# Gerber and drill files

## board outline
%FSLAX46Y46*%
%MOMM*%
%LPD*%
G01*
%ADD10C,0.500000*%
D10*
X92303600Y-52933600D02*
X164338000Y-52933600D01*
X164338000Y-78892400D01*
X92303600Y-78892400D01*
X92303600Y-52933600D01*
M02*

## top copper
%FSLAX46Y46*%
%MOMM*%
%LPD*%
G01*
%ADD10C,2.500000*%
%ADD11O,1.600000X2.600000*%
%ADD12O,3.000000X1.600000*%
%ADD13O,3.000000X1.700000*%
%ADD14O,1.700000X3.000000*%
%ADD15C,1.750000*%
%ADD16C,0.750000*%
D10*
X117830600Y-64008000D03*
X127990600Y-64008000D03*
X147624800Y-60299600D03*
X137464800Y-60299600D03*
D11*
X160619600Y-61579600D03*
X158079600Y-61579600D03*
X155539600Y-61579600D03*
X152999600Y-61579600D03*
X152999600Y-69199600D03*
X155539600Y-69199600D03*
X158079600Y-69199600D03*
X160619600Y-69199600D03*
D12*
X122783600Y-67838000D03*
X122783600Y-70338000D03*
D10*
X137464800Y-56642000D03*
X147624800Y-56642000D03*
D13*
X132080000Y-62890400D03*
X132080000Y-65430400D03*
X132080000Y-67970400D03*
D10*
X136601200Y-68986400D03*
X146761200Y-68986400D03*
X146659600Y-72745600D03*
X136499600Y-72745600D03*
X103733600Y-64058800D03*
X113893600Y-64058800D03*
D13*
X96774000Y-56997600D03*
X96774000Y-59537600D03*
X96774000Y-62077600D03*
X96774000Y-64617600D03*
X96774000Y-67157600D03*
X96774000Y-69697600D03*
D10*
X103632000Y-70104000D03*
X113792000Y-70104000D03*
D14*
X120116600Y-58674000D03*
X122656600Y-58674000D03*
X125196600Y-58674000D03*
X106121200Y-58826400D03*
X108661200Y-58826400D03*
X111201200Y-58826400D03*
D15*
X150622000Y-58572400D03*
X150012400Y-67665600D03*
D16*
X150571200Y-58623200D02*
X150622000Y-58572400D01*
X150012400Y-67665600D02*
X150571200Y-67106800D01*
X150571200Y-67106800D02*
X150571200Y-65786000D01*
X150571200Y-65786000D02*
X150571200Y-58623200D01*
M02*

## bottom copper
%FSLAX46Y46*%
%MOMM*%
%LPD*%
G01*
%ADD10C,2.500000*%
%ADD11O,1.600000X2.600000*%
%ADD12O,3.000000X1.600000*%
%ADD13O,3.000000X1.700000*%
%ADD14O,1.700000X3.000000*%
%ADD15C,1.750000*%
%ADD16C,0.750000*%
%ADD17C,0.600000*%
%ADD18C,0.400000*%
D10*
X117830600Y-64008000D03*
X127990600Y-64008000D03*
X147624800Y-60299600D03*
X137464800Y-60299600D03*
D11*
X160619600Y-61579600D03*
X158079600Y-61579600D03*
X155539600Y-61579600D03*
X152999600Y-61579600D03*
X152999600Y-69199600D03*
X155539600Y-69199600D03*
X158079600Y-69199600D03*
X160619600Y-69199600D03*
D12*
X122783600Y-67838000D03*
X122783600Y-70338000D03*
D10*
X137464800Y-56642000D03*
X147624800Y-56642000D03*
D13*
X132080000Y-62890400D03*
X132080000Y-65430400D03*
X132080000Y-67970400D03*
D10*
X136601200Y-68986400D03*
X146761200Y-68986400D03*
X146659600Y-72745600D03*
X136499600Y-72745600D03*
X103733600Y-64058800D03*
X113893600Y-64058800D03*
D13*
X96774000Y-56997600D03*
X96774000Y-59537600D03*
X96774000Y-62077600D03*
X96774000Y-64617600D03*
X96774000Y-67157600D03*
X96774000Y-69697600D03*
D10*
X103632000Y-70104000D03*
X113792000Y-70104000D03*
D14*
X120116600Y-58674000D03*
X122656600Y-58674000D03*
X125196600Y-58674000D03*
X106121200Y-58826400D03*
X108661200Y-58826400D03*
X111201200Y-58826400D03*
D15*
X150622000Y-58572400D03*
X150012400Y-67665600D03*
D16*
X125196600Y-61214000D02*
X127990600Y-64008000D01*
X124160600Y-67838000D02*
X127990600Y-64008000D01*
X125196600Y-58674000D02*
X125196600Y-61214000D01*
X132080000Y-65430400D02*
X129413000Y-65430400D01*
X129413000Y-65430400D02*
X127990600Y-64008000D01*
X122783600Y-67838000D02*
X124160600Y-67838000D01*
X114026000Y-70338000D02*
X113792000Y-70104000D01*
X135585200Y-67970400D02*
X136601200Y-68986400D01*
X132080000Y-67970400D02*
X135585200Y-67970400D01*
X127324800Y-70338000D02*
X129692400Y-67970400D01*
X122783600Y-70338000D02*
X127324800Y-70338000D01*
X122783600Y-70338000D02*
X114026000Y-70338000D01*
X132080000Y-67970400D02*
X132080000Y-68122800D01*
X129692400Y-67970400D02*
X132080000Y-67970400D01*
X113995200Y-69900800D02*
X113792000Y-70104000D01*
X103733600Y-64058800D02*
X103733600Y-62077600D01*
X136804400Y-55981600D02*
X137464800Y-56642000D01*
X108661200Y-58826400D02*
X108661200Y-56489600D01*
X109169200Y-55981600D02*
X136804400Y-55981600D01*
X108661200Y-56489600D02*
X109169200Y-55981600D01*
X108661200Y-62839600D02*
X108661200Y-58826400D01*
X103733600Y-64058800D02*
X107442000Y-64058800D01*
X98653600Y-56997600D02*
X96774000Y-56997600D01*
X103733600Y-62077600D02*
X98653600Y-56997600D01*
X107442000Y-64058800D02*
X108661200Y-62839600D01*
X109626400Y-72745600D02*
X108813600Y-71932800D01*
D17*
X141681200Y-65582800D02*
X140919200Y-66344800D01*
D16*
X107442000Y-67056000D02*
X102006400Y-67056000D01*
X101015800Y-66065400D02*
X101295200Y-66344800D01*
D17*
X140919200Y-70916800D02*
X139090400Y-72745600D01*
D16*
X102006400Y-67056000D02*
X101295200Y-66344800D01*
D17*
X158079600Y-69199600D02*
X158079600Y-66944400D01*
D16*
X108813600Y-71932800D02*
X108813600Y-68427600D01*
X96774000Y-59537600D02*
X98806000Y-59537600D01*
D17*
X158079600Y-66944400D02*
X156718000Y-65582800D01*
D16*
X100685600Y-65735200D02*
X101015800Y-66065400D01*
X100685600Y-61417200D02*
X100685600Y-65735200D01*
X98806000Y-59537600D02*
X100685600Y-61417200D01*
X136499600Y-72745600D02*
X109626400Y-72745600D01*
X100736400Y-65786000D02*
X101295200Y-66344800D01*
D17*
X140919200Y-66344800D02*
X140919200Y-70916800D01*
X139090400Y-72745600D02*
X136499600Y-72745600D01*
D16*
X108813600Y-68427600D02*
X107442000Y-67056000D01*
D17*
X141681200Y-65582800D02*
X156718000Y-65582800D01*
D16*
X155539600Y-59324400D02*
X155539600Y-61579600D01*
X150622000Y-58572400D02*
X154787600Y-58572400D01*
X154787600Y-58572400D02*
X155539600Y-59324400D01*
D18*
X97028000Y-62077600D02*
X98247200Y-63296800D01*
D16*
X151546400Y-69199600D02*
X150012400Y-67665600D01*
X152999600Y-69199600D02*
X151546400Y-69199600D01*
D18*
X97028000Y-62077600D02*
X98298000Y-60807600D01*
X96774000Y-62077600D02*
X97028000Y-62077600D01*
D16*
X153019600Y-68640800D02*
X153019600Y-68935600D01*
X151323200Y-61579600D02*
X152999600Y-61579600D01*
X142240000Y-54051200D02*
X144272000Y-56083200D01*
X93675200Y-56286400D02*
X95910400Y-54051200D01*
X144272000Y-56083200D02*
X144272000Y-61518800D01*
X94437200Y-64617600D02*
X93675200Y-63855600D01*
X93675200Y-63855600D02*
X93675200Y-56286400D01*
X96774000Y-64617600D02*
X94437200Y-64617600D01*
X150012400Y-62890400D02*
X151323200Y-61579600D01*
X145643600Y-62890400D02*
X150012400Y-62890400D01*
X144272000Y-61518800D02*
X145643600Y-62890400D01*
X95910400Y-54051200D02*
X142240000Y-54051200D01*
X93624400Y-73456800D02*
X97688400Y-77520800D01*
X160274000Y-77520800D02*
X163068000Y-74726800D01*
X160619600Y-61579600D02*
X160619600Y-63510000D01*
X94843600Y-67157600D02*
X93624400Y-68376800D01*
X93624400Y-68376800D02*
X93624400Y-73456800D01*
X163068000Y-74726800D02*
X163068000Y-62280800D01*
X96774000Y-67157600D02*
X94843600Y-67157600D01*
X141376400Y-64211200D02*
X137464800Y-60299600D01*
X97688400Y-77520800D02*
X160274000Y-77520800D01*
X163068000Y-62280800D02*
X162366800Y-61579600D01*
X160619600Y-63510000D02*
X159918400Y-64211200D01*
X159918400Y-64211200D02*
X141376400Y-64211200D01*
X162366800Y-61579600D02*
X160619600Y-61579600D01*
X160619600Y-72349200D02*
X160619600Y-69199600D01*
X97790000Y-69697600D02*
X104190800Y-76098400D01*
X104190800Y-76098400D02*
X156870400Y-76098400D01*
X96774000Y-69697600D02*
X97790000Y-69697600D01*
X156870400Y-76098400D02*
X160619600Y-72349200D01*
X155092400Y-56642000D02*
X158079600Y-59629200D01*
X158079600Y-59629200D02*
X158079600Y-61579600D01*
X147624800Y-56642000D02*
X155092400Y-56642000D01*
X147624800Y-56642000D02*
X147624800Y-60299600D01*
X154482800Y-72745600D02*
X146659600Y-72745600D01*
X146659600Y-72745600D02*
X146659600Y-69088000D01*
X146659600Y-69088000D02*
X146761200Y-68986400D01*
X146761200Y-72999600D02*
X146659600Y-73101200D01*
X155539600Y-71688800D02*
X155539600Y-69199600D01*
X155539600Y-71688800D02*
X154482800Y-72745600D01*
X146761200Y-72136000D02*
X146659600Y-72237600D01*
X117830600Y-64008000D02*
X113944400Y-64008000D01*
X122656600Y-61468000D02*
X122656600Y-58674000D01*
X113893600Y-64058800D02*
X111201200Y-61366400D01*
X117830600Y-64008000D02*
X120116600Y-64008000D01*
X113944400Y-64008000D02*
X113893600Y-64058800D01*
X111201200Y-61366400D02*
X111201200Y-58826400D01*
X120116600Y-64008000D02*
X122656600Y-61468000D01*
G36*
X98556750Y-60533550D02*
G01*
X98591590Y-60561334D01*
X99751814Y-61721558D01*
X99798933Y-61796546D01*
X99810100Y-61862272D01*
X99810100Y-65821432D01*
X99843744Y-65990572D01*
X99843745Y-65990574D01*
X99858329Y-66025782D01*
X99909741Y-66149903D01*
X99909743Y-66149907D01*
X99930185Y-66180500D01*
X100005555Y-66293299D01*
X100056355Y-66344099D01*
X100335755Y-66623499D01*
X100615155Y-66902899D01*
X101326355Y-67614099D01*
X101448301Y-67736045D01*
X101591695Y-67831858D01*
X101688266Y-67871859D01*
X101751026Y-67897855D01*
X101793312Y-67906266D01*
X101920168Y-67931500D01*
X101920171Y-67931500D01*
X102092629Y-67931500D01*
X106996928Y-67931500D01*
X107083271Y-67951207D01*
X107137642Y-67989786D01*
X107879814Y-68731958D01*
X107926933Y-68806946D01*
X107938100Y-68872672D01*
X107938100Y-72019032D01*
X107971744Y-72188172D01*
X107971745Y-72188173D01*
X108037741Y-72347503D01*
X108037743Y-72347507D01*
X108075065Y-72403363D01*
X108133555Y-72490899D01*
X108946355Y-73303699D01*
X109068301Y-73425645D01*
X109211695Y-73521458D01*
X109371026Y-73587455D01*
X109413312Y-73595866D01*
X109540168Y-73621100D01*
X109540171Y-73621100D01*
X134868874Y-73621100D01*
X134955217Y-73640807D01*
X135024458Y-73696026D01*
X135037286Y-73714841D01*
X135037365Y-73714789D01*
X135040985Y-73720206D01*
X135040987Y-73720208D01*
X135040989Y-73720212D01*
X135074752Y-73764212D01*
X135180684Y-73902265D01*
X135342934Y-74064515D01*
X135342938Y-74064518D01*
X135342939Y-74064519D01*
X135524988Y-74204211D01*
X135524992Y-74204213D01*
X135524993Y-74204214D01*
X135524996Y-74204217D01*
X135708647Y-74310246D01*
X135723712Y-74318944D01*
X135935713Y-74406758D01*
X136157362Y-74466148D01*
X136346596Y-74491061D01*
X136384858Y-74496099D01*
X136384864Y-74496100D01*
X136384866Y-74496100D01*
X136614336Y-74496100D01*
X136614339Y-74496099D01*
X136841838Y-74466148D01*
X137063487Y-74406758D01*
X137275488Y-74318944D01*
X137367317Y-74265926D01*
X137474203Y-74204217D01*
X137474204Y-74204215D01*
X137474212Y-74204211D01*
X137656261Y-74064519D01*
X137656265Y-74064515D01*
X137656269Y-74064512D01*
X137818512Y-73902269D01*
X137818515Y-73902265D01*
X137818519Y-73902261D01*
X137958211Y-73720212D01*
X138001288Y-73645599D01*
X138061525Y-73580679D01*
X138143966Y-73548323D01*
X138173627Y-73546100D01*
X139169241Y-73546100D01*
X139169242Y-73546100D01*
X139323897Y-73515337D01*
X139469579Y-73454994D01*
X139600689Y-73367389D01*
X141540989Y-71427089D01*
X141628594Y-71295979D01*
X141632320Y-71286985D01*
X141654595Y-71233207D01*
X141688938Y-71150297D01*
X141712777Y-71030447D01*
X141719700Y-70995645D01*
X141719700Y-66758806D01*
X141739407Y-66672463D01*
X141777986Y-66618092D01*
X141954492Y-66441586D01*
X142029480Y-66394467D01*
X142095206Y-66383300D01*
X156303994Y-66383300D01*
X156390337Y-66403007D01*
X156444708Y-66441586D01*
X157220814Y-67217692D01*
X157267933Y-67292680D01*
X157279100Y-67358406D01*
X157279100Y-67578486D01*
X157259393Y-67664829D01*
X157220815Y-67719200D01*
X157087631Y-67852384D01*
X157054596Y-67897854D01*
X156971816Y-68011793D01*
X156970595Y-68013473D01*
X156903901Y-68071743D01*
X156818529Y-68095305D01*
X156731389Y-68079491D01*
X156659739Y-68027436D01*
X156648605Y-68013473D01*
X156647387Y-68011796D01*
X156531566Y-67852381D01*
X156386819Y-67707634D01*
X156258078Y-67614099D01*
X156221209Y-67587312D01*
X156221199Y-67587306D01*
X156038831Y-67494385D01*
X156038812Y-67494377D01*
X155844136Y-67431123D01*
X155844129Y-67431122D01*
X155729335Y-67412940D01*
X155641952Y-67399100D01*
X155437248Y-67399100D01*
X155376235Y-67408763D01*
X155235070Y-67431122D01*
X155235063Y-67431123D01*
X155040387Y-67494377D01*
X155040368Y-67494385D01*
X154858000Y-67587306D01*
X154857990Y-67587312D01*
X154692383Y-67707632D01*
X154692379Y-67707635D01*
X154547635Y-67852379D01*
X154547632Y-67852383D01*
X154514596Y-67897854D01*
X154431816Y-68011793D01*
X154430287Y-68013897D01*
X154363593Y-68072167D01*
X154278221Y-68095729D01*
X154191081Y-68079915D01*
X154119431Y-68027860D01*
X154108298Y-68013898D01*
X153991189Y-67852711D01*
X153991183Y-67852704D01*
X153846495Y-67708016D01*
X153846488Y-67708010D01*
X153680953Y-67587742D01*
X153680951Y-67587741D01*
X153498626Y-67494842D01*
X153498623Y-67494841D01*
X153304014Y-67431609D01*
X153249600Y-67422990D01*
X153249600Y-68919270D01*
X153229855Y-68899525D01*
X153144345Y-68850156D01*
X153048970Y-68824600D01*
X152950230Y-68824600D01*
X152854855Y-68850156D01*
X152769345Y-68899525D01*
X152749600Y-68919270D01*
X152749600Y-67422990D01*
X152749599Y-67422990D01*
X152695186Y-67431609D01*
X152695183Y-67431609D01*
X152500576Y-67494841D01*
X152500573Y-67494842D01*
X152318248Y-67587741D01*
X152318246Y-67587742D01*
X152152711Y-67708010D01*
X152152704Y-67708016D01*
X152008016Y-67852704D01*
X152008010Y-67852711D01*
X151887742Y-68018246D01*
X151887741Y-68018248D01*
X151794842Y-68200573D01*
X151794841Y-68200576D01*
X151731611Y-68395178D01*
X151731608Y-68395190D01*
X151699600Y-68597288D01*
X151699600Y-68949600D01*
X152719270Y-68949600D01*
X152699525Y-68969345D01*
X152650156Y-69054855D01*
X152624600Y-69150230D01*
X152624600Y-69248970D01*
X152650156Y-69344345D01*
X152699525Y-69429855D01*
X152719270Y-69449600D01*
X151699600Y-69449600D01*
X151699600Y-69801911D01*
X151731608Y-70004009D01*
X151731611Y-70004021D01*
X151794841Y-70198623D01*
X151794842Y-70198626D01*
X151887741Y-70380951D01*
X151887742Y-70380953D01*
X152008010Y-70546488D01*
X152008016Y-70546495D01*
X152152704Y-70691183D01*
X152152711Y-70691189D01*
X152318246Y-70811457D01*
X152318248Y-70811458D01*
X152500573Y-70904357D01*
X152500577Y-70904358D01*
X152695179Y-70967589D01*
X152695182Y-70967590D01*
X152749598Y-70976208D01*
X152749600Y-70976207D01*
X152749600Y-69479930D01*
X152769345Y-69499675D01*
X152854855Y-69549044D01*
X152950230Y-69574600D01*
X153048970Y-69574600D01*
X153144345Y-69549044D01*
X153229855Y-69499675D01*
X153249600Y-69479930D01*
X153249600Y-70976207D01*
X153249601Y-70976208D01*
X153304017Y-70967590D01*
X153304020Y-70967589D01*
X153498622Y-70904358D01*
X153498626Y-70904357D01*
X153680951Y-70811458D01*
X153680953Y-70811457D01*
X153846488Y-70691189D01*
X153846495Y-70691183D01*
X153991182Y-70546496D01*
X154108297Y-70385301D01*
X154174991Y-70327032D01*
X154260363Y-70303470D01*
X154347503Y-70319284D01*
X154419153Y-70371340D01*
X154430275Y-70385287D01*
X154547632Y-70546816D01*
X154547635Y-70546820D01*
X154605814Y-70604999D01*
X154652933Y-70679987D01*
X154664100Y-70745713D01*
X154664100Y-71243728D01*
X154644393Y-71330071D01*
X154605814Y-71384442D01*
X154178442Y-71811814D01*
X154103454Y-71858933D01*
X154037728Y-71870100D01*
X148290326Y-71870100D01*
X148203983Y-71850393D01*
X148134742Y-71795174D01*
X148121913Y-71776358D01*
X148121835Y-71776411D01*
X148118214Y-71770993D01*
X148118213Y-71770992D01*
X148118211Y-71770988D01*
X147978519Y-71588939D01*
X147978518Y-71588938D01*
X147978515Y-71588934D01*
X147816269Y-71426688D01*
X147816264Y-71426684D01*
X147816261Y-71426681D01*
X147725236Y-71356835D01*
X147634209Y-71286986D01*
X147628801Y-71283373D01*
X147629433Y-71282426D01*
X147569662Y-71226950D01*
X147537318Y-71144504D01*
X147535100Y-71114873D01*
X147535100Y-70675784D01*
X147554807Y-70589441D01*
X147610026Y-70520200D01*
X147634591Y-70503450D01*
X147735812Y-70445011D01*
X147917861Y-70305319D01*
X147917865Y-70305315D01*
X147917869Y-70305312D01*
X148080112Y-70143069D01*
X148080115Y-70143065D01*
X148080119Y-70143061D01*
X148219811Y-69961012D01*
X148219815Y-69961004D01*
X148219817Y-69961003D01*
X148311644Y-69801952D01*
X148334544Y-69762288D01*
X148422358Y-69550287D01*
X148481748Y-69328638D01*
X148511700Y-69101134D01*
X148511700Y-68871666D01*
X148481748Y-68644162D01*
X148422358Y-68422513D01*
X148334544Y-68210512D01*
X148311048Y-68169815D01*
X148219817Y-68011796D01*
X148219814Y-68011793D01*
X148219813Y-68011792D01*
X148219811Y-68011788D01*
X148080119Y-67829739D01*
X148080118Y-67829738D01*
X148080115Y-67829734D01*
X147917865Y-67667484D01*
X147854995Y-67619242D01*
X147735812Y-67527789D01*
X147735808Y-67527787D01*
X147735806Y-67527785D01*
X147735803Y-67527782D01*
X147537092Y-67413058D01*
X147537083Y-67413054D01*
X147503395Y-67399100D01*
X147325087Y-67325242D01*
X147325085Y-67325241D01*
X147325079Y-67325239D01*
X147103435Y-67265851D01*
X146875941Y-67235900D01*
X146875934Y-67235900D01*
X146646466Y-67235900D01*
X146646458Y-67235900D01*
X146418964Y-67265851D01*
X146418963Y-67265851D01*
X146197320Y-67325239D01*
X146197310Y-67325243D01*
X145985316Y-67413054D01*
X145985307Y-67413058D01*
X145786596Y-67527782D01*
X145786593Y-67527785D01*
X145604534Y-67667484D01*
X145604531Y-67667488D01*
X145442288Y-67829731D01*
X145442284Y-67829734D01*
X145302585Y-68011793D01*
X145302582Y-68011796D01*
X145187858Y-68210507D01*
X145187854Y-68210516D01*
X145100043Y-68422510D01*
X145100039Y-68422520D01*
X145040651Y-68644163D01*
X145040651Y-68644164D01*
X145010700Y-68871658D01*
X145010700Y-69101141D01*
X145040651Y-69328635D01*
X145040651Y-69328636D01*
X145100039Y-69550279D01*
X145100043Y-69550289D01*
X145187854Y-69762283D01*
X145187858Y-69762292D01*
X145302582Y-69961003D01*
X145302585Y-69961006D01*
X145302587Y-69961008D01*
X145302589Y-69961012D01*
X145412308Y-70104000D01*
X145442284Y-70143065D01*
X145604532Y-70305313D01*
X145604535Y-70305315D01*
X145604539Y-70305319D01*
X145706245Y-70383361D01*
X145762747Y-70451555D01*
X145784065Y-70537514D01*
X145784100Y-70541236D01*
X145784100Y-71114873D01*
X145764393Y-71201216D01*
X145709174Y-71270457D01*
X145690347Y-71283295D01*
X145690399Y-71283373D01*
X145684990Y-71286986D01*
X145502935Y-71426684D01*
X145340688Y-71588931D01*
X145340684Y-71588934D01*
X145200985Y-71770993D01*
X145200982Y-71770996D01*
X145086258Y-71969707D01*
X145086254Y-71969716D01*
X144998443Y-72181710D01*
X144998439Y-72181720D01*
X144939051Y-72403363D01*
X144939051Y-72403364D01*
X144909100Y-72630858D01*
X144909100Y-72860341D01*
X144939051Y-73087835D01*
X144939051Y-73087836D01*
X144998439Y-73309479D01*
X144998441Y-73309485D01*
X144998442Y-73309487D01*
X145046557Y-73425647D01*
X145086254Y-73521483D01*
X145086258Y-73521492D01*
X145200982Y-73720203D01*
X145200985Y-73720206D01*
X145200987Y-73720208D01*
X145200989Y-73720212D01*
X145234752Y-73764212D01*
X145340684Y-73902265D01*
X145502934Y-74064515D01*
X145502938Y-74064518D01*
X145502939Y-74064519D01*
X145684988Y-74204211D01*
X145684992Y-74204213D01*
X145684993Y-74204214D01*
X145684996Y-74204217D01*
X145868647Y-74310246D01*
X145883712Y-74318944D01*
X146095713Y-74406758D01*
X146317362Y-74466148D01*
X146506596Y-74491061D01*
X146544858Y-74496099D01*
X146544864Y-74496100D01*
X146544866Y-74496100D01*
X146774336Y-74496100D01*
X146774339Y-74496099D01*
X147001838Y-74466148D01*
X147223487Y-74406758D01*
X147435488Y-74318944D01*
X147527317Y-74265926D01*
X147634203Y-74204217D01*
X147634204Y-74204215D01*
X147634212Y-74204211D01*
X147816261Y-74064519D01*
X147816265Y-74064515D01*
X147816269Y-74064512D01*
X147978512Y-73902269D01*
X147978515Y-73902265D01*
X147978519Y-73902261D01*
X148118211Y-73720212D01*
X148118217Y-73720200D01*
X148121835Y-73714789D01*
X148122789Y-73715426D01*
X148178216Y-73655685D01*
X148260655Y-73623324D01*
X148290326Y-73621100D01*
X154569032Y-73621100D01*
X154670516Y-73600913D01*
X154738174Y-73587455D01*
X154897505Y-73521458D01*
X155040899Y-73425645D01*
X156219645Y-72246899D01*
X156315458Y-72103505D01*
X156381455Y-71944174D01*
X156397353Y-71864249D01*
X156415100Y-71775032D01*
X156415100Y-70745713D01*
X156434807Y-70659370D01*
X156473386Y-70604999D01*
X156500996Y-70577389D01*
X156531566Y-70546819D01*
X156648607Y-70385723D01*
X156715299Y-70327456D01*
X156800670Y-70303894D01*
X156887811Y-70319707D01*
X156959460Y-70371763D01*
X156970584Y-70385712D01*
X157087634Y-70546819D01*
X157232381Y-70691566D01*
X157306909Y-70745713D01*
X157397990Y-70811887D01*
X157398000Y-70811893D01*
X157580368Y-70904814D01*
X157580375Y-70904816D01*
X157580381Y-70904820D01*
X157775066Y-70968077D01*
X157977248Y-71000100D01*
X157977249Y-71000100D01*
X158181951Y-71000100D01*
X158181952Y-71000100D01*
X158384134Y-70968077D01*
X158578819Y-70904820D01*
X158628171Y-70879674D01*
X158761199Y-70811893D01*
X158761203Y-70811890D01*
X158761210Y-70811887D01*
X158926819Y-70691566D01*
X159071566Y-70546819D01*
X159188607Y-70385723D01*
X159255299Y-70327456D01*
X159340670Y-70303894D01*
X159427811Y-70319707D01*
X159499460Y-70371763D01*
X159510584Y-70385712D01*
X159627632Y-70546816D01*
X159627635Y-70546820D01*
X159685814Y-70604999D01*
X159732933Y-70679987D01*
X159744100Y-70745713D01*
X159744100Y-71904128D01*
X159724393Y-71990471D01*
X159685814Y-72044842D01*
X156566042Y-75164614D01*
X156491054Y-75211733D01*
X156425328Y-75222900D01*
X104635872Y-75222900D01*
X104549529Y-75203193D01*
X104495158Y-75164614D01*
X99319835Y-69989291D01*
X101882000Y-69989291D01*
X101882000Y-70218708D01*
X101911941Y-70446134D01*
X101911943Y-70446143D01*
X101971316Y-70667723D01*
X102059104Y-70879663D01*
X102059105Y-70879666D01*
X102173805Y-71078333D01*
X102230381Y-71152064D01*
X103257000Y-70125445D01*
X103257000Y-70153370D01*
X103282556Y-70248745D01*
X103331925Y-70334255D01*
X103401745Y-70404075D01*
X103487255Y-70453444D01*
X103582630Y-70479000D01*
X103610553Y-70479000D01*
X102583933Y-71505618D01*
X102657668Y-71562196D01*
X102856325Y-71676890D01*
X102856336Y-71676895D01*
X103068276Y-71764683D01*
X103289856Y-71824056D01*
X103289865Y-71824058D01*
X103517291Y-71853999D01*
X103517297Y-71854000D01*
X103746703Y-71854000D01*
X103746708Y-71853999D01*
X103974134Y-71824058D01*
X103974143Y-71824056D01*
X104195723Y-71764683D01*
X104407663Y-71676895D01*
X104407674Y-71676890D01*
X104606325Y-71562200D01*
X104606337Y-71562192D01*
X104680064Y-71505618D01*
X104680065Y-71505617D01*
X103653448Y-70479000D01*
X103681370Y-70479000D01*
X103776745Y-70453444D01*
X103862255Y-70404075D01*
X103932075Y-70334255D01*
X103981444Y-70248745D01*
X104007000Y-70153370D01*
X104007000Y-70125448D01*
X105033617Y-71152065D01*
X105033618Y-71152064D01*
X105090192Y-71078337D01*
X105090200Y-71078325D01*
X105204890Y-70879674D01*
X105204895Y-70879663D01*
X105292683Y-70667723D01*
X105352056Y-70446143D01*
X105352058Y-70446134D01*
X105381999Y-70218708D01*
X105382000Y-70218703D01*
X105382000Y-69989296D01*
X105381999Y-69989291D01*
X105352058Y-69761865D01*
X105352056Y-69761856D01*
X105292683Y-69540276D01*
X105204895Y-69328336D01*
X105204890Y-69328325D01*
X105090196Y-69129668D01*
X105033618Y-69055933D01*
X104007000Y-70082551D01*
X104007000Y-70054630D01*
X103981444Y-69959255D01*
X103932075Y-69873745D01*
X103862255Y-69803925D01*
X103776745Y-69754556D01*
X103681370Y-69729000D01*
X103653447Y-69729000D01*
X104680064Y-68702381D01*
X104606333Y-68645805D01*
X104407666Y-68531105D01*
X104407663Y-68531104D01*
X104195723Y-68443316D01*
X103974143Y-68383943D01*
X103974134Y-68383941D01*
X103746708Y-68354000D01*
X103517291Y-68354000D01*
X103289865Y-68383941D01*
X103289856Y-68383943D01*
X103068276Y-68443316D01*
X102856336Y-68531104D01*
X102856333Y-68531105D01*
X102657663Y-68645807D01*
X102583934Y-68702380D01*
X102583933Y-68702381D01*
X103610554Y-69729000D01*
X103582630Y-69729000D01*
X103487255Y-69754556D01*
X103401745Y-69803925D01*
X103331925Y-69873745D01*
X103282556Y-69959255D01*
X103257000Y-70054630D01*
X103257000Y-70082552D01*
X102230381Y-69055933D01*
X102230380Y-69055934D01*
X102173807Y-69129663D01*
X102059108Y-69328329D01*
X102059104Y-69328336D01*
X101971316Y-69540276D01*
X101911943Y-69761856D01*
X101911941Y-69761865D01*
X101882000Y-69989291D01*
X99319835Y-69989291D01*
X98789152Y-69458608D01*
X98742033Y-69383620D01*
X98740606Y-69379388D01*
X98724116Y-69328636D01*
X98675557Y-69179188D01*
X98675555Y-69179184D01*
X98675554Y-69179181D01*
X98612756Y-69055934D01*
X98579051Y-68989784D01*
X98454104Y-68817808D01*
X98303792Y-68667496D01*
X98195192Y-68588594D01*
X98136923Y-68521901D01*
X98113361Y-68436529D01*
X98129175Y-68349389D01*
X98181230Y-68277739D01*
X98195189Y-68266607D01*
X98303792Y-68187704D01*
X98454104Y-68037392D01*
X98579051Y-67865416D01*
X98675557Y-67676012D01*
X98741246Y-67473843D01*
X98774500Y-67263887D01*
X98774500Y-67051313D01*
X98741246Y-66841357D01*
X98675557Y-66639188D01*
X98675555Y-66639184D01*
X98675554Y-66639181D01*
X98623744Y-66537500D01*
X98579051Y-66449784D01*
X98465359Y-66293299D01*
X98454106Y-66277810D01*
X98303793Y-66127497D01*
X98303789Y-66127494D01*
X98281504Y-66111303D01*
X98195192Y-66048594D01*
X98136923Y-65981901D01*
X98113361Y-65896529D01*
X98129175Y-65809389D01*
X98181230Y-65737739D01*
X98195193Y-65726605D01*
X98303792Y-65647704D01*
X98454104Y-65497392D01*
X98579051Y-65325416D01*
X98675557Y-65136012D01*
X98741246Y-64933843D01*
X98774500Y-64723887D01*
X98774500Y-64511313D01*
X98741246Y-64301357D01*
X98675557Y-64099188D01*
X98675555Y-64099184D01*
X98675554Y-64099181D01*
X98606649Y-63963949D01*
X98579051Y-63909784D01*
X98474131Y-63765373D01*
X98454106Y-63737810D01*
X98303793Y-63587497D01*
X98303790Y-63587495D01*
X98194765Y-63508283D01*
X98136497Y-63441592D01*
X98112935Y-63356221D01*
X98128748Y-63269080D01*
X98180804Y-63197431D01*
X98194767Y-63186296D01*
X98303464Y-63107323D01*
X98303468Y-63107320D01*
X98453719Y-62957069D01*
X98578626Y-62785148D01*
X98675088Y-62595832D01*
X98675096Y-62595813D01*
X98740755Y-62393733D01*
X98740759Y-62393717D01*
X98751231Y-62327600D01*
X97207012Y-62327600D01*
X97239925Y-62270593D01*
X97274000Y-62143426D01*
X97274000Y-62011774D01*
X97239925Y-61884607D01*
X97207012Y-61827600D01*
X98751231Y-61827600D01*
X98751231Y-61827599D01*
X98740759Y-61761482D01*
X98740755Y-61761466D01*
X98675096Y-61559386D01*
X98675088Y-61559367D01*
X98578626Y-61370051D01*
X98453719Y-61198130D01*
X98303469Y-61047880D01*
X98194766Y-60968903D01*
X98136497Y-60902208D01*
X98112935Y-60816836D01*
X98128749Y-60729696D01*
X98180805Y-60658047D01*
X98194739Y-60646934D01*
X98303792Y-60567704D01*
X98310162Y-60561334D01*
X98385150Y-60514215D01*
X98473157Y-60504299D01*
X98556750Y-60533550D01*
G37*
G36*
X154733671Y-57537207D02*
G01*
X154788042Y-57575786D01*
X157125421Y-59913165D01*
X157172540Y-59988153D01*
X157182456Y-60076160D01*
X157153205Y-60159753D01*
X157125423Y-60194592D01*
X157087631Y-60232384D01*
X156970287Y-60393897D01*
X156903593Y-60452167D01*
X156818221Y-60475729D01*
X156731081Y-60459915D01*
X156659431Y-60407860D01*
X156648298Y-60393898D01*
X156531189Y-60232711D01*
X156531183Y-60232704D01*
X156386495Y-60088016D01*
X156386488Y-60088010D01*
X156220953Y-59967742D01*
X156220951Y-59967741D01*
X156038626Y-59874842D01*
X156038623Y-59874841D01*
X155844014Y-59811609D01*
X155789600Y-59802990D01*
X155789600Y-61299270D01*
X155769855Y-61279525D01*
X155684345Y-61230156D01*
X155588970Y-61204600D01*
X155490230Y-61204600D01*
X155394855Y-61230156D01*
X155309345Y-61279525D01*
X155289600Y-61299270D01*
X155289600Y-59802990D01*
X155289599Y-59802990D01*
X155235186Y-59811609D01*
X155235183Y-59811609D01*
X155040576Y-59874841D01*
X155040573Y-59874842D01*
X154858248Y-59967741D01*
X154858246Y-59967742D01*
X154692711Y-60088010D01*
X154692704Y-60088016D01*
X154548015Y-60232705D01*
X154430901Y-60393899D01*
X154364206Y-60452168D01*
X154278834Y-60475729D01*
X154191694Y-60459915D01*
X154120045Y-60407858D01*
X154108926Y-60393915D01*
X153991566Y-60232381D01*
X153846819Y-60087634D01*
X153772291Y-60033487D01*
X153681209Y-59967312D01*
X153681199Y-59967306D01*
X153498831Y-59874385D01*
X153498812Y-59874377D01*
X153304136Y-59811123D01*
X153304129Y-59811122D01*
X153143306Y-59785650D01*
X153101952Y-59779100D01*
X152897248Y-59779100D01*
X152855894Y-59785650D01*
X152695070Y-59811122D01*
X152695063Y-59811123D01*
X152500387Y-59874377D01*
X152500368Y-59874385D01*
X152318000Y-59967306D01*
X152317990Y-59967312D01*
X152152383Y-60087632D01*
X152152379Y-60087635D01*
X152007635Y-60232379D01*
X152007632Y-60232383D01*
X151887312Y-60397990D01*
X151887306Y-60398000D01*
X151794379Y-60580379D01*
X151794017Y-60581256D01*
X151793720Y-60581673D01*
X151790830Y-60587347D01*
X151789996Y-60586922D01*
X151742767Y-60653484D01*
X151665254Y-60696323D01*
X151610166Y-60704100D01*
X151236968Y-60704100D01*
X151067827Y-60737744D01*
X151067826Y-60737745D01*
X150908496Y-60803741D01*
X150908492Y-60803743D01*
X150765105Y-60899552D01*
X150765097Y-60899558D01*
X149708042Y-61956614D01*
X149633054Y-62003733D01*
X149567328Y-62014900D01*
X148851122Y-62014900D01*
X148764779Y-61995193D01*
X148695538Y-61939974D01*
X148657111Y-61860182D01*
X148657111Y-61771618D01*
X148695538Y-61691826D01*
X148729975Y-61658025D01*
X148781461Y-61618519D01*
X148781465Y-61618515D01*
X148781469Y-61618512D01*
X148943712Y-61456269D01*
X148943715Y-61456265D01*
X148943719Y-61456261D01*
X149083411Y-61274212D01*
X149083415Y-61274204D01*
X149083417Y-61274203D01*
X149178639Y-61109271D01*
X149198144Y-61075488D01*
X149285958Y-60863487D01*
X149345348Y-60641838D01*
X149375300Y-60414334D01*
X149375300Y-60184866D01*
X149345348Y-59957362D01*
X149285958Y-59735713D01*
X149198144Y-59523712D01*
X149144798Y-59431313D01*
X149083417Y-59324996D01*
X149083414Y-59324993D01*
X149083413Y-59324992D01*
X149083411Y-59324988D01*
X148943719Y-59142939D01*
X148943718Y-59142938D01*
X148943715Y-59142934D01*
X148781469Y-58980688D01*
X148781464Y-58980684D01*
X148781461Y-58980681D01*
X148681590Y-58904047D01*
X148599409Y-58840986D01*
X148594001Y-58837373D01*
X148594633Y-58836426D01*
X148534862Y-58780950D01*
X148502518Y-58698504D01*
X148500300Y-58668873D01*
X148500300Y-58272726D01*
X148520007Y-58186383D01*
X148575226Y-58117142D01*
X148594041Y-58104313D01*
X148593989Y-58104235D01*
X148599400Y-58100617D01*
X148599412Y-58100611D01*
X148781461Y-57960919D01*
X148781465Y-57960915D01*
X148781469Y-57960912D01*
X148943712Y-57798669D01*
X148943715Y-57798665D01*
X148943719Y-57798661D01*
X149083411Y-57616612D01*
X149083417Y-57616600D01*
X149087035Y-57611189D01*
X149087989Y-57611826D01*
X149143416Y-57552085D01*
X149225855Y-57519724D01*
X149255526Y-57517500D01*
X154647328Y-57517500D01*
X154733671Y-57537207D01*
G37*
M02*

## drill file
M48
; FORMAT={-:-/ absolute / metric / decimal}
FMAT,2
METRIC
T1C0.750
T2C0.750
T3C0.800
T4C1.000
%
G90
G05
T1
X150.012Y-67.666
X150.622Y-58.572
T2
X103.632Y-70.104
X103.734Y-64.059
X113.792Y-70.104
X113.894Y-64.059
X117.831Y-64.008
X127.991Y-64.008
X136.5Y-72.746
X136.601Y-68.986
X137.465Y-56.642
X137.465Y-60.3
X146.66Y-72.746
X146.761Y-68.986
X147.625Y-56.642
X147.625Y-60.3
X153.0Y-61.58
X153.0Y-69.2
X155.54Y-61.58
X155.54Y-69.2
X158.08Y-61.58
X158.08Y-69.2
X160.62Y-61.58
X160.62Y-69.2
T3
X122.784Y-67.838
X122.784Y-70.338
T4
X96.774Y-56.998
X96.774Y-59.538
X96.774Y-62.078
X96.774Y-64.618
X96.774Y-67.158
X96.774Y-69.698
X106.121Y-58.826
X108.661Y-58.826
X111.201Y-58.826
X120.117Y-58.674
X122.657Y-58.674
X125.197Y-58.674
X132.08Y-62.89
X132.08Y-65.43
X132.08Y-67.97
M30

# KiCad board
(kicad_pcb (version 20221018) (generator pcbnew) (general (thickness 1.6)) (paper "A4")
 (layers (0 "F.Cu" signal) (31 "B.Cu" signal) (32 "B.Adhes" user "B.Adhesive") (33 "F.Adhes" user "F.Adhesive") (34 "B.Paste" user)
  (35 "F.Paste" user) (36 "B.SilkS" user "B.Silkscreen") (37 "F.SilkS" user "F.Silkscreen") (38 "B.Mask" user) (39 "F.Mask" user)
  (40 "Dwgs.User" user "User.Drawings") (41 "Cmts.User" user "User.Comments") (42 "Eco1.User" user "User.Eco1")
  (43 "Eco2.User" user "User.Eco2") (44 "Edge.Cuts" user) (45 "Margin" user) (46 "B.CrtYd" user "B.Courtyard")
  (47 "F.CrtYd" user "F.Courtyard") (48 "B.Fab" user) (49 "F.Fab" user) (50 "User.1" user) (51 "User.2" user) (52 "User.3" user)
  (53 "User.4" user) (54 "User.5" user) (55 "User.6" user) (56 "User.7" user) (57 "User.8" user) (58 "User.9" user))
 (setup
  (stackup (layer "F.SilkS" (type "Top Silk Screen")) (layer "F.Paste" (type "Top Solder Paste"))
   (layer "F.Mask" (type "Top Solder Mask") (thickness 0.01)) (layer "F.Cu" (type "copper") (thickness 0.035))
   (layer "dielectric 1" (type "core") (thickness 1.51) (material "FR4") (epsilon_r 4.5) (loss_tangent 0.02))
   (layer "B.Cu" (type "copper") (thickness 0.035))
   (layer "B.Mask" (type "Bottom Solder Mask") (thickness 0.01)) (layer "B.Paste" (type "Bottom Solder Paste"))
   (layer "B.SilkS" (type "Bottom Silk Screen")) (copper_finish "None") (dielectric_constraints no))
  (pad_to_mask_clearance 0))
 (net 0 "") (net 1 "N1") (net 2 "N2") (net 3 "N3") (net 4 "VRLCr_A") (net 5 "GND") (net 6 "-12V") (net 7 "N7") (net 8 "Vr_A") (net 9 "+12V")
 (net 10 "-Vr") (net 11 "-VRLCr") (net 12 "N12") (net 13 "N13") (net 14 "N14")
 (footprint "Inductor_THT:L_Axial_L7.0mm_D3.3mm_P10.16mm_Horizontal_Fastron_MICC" (layer "F.Cu") (at 117.8306 64.008)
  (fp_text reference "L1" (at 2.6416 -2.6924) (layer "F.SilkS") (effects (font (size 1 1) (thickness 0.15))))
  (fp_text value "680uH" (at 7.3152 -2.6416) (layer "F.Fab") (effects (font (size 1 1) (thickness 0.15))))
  (pad "1" thru_hole circle (at 0 0) (size 2.5 2.5) (drill 0.75) (layers "*.Cu" "*.Mask") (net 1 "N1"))
  (pad "2" thru_hole circle (at 10.16 0) (size 2.5 2.5) (drill 0.75) (layers "*.Cu" "*.Mask") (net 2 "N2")))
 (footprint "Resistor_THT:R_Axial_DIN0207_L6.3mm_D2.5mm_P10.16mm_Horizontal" (layer "F.Cu") (at 147.6248 60.2996 180)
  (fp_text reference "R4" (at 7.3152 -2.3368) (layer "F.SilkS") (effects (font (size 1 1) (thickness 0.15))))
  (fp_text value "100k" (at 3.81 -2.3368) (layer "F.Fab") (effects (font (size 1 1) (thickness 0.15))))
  (pad "1" thru_hole circle (at 0 0 180) (size 2.5 2.5) (drill 0.75) (layers "*.Cu" "*.Mask") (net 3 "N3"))
  (pad "2" thru_hole circle (at 10.16 0 180) (size 2.5 2.5) (drill 0.75) (layers "*.Cu" "*.Mask") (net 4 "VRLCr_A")))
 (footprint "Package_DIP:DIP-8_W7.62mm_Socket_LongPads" (layer "F.Cu") (at 160.6196 61.5796 -90)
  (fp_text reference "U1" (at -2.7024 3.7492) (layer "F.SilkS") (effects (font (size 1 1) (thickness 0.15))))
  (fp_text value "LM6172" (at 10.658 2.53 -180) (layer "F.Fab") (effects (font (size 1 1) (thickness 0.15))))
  (pad "1" thru_hole oval (at 0 0 270) (size 2.6 1.6) (drill 0.75) (layers "*.Cu" "*.Mask") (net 4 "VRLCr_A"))
  (pad "2" thru_hole oval (at 0 2.54 270) (size 2.6 1.6) (drill 0.75) (layers "*.Cu" "*.Mask") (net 3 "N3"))
  (pad "3" thru_hole oval (at 0 5.08 270) (size 2.6 1.6) (drill 0.75) (layers "*.Cu" "*.Mask") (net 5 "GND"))
  (pad "4" thru_hole oval (at 0 7.62 270) (size 2.6 1.6) (drill 0.75) (layers "*.Cu" "*.Mask") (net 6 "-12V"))
  (pad "5" thru_hole oval (at 7.62 7.62 270) (size 2.6 1.6) (drill 0.75) (layers "*.Cu" "*.Mask") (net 5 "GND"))
  (pad "6" thru_hole oval (at 7.62 5.08 270) (size 2.6 1.6) (drill 0.75) (layers "*.Cu" "*.Mask") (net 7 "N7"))
  (pad "7" thru_hole oval (at 7.62 2.54 270) (size 2.6 1.6) (drill 0.75) (layers "*.Cu" "*.Mask") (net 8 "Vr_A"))
  (pad "8" thru_hole oval (at 7.62 0 270) (size 2.6 1.6) (drill 0.75) (layers "*.Cu" "*.Mask") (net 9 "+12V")))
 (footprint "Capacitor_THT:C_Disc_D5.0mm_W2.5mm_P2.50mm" (layer "F.Cu") (at 122.7836 67.838 -90)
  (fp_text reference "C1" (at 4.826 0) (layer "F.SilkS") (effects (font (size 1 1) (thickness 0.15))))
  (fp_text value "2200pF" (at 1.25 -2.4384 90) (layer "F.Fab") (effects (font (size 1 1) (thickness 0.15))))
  (pad "1" thru_hole oval (at 0 0 270) (size 1.6 3) (drill 0.8) (layers "*.Cu" "*.Mask") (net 2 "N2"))
  (pad "2" thru_hole oval (at 2.5 0 270) (size 1.6 3) (drill 0.8) (layers "*.Cu" "*.Mask") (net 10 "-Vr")))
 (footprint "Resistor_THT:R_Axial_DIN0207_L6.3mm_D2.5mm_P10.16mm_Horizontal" (layer "F.Cu") (at 137.4648 56.642)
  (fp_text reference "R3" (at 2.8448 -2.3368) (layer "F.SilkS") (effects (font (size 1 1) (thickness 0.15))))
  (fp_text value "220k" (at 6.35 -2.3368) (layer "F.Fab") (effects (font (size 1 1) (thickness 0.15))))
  (pad "1" thru_hole circle (at 0 0) (size 2.5 2.5) (drill 0.75) (layers "*.Cu" "*.Mask") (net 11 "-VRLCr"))
  (pad "2" thru_hole circle (at 10.16 0) (size 2.5 2.5) (drill 0.75) (layers "*.Cu" "*.Mask") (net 3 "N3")))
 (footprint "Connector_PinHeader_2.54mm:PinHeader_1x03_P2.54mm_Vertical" (layer "F.Cu") (at 132.08 62.8904)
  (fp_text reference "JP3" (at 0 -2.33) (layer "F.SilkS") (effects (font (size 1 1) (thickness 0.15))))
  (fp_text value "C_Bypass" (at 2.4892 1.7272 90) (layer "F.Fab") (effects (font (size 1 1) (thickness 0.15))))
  (pad "1" thru_hole oval (at 0 0) (size 3 1.7) (drill 1) (layers "*.Cu" "*.Mask") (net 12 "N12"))
  (pad "2" thru_hole oval (at 0 2.54) (size 3 1.7) (drill 1) (layers "*.Cu" "*.Mask") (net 2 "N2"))
  (pad "3" thru_hole oval (at 0 5.08) (size 3 1.7) (drill 1) (layers "*.Cu" "*.Mask") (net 10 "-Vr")))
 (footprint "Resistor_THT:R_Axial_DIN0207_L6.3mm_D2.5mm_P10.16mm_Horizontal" (layer "F.Cu") (at 136.6012 68.9864)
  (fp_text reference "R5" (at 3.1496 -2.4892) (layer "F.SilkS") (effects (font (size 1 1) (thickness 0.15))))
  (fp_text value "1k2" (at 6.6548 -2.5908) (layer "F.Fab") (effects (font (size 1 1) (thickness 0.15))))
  (pad "1" thru_hole circle (at 0 0) (size 2.5 2.5) (drill 0.75) (layers "*.Cu" "*.Mask") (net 10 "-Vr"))
  (pad "2" thru_hole circle (at 10.16 0) (size 2.5 2.5) (drill 0.75) (layers "*.Cu" "*.Mask") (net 7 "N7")))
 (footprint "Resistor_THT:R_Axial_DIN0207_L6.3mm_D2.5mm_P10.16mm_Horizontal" (layer "F.Cu") (at 146.6596 72.7456 180)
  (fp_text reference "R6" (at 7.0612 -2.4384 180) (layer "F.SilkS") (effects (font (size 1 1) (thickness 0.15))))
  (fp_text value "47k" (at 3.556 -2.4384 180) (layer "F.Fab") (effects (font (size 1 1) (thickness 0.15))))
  (pad "1" thru_hole circle (at 0 0 180) (size 2.5 2.5) (drill 0.75) (layers "*.Cu" "*.Mask") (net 7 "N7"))
  (pad "2" thru_hole circle (at 10.16 0 180) (size 2.5 2.5) (drill 0.75) (layers "*.Cu" "*.Mask") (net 8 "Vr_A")))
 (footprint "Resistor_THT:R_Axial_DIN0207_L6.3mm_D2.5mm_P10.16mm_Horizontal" (layer "F.Cu") (at 103.7336 64.0588)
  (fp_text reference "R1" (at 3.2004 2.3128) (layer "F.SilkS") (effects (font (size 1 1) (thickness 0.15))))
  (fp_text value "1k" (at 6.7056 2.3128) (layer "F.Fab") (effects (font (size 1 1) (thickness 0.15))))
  (pad "1" thru_hole circle (at 0 0) (size 2.5 2.5) (drill 0.75) (layers "*.Cu" "*.Mask") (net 11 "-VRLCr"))
  (pad "2" thru_hole circle (at 10.16 0) (size 2.5 2.5) (drill 0.75) (layers "*.Cu" "*.Mask") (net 1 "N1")))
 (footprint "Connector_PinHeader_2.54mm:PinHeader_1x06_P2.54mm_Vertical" (layer "F.Cu") (at 96.774 56.9976)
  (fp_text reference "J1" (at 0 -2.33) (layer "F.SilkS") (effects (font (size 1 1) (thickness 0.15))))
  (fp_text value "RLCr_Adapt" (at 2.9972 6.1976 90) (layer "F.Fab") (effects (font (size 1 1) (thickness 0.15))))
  (pad "1" thru_hole oval (at 0 0) (size 3 1.7) (drill 1) (layers "*.Cu" "*.Mask") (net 11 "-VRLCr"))
  (pad "2" thru_hole oval (at 0 2.54) (size 3 1.7) (drill 1) (layers "*.Cu" "*.Mask") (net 8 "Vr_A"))
  (pad "3" thru_hole oval (at 0 5.08) (size 3 1.7) (drill 1) (layers "*.Cu" "*.Mask") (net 5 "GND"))
  (pad "4" thru_hole oval (at 0 7.62) (size 3 1.7) (drill 1) (layers "*.Cu" "*.Mask") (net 6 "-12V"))
  (pad "5" thru_hole oval (at 0 10.16) (size 3 1.7) (drill 1) (layers "*.Cu" "*.Mask") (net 4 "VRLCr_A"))
  (pad "6" thru_hole oval (at 0 12.7) (size 3 1.7) (drill 1) (layers "*.Cu" "*.Mask") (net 9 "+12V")))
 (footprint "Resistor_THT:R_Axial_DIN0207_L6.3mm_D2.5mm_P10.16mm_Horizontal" (layer "F.Cu") (at 103.632 70.104)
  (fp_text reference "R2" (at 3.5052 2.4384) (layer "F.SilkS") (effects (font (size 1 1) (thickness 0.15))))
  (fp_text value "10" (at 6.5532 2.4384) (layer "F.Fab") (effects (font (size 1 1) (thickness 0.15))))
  (pad "1" thru_hole circle (at 0 0) (size 2.5 2.5) (drill 0.75) (layers "*.Cu" "*.Mask") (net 5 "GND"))
  (pad "2" thru_hole circle (at 10.16 0) (size 2.5 2.5) (drill 0.75) (layers "*.Cu" "*.Mask") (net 10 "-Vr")))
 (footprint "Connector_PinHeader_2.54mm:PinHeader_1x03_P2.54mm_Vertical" (layer "F.Cu") (at 120.1166 58.674 90)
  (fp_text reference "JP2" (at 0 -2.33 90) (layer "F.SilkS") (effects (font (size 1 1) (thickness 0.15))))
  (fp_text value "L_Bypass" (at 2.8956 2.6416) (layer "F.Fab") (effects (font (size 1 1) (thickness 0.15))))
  (pad "1" thru_hole oval (at 0 0 90) (size 3 1.7) (drill 1) (layers "*.Cu" "*.Mask") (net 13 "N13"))
  (pad "2" thru_hole oval (at 0 2.54 90) (size 3 1.7) (drill 1) (layers "*.Cu" "*.Mask") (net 1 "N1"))
  (pad "3" thru_hole oval (at 0 5.08 90) (size 3 1.7) (drill 1) (layers "*.Cu" "*.Mask") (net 2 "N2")))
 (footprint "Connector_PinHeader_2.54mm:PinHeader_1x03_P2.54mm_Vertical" (layer "F.Cu") (at 106.1212 58.8264 90)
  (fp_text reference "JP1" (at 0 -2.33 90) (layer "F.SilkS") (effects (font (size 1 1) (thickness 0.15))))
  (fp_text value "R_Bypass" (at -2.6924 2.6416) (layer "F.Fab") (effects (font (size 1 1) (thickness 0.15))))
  (pad "1" thru_hole oval (at 0 0 90) (size 3 1.7) (drill 1) (layers "*.Cu" "*.Mask") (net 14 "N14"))
  (pad "2" thru_hole oval (at 0 2.54 90) (size 3 1.7) (drill 1) (layers "*.Cu" "*.Mask") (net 11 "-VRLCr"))
  (pad "3" thru_hole oval (at 0 5.08 90) (size 3 1.7) (drill 1) (layers "*.Cu" "*.Mask") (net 1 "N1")))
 (gr_rect (start 92.3036 52.9336) (end 164.338 78.8924) (stroke (width 0.5) (type default)) (fill none) (layer "Edge.Cuts"))
 (segment (start 125.1966 61.214) (end 127.9906 64.008) (width 0.75) (layer "B.Cu") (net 2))
 (segment (start 124.1606 67.838) (end 127.9906 64.008) (width 0.75) (layer "B.Cu") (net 2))
 (segment (start 125.1966 58.674) (end 125.1966 61.214) (width 0.75) (layer "B.Cu") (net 2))
 (segment (start 132.08 65.4304) (end 129.413 65.4304) (width 0.75) (layer "B.Cu") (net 2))
 (segment (start 129.413 65.4304) (end 127.9906 64.008) (width 0.75) (layer "B.Cu") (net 2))
 (segment (start 122.7836 67.838) (end 124.1606 67.838) (width 0.75) (layer "B.Cu") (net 2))
 (segment (start 114.026 70.338) (end 113.792 70.104) (width 0.75) (layer "B.Cu") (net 10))
 (segment (start 135.5852 67.9704) (end 136.6012 68.9864) (width 0.75) (layer "B.Cu") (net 10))
 (segment (start 132.08 67.9704) (end 135.5852 67.9704) (width 0.75) (layer "B.Cu") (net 10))
 (segment (start 127.3248 70.338) (end 129.6924 67.9704) (width 0.75) (layer "B.Cu") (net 10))
 (segment (start 122.7836 70.338) (end 127.3248 70.338) (width 0.75) (layer "B.Cu") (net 10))
 (segment (start 122.7836 70.338) (end 114.026 70.338) (width 0.75) (layer "B.Cu") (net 10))
 (segment (start 132.08 67.9704) (end 132.08 68.1228) (width 0.75) (layer "B.Cu") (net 10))
 (segment (start 129.6924 67.9704) (end 132.08 67.9704) (width 0.75) (layer "B.Cu") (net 10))
 (segment (start 113.9952 69.9008) (end 113.792 70.104) (width 0.75) (layer "B.Cu") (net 10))
 (segment (start 103.7336 64.0588) (end 103.7336 62.0776) (width 0.75) (layer "B.Cu") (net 11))
 (segment (start 136.8044 55.9816) (end 137.4648 56.642) (width 0.75) (layer "B.Cu") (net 11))
 (segment (start 108.6612 58.8264) (end 108.6612 56.4896) (width 0.75) (layer "B.Cu") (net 11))
 (segment (start 109.1692 55.9816) (end 136.8044 55.9816) (width 0.75) (layer "B.Cu") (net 11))
 (segment (start 108.6612 56.4896) (end 109.1692 55.9816) (width 0.75) (layer "B.Cu") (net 11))
 (segment (start 108.6612 62.8396) (end 108.6612 58.8264) (width 0.75) (layer "B.Cu") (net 11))
 (segment (start 103.7336 64.0588) (end 107.442 64.0588) (width 0.75) (layer "B.Cu") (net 11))
 (segment (start 98.6536 56.9976) (end 96.774 56.9976) (width 0.75) (layer "B.Cu") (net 11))
 (segment (start 103.7336 62.0776) (end 98.6536 56.9976) (width 0.75) (layer "B.Cu") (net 11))
 (segment (start 107.442 64.0588) (end 108.6612 62.8396) (width 0.75) (layer "B.Cu") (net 11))
 (segment (start 109.6264 72.7456) (end 108.8136 71.9328) (width 0.75) (layer "B.Cu") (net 8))
 (segment (start 141.6812 65.5828) (end 140.9192 66.3448) (width 0.6) (layer "B.Cu") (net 8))
 (segment (start 107.442 67.056) (end 102.0064 67.056) (width 0.75) (layer "B.Cu") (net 8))
 (segment (start 101.0158 66.0654) (end 101.2952 66.3448) (width 0.75) (layer "B.Cu") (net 8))
 (segment (start 140.9192 70.9168) (end 139.0904 72.7456) (width 0.6) (layer "B.Cu") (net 8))
 (segment (start 102.0064 67.056) (end 101.2952 66.3448) (width 0.75) (layer "B.Cu") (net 8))
 (segment (start 158.0796 69.1996) (end 158.0796 66.9444) (width 0.6) (layer "B.Cu") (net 8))
 (segment (start 108.8136 71.9328) (end 108.8136 68.4276) (width 0.75) (layer "B.Cu") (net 8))
 (segment (start 96.774 59.5376) (end 98.806 59.5376) (width 0.75) (layer "B.Cu") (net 8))
 (segment (start 158.0796 66.9444) (end 156.718 65.5828) (width 0.6) (layer "B.Cu") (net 8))
 (segment (start 100.6856 65.7352) (end 101.0158 66.0654) (width 0.75) (layer "B.Cu") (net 8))
 (segment (start 100.6856 61.4172) (end 100.6856 65.7352) (width 0.75) (layer "B.Cu") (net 8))
 (segment (start 98.806 59.5376) (end 100.6856 61.4172) (width 0.75) (layer "B.Cu") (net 8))
 (segment (start 136.4996 72.7456) (end 109.6264 72.7456) (width 0.75) (layer "B.Cu") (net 8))
 (segment (start 100.7364 65.786) (end 101.2952 66.3448) (width 0.75) (layer "B.Cu") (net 8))
 (segment (start 140.9192 66.3448) (end 140.9192 70.9168) (width 0.6) (layer "B.Cu") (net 8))
 (segment (start 139.0904 72.7456) (end 136.4996 72.7456) (width 0.6) (layer "B.Cu") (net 8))
 (segment (start 108.8136 68.4276) (end 107.442 67.056) (width 0.75) (layer "B.Cu") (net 8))
 (segment (start 141.6812 65.5828) (end 156.718 65.5828) (width 0.6) (layer "B.Cu") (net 8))
 (segment (start 150.5712 58.6232) (end 150.622 58.5724) (width 0.75) (layer "F.Cu") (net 5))
 (segment (start 150.0124 67.6656) (end 150.5712 67.1068) (width 0.75) (layer "F.Cu") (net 5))
 (segment (start 150.5712 67.1068) (end 150.5712 65.786) (width 0.75) (layer "F.Cu") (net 5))
 (segment (start 150.5712 65.786) (end 150.5712 58.6232) (width 0.75) (layer "F.Cu") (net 5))
 (via (at 150.622 58.5724) (size 1.75) (drill 0.75) (layers "F.Cu" "B.Cu") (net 5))
 (via (at 150.0124 67.6656) (size 1.75) (drill 0.75) (layers "F.Cu" "B.Cu") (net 5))
 (segment (start 155.5396 59.3244) (end 155.5396 61.5796) (width 0.75) (layer "B.Cu") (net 5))
 (segment (start 150.622 58.5724) (end 154.7876 58.5724) (width 0.75) (layer "B.Cu") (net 5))
 (segment (start 154.7876 58.5724) (end 155.5396 59.3244) (width 0.75) (layer "B.Cu") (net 5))
 (segment (start 97.028 62.0776) (end 98.2472 63.2968) (width 0.4) (layer "B.Cu") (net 5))
 (segment (start 151.5464 69.1996) (end 150.0124 67.6656) (width 0.75) (layer "B.Cu") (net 5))
 (segment (start 152.9996 69.1996) (end 151.5464 69.1996) (width 0.75) (layer "B.Cu") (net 5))
 (segment (start 97.028 62.0776) (end 98.298 60.8076) (width 0.4) (layer "B.Cu") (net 5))
 (segment (start 96.774 62.0776) (end 97.028 62.0776) (width 0.4) (layer "B.Cu") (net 5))
 (segment (start 153.0196 68.6408) (end 153.0196 68.9356) (width 0.75) (layer "B.Cu") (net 5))
 (segment (start 151.3232 61.5796) (end 152.9996 61.5796) (width 0.75) (layer "B.Cu") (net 6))
 (segment (start 142.24 54.0512) (end 144.272 56.0832) (width 0.75) (layer "B.Cu") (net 6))
 (segment (start 93.6752 56.2864) (end 95.9104 54.0512) (width 0.75) (layer "B.Cu") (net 6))
 (segment (start 144.272 56.0832) (end 144.272 61.5188) (width 0.75) (layer "B.Cu") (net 6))
 (segment (start 94.4372 64.6176) (end 93.6752 63.8556) (width 0.75) (layer "B.Cu") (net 6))
 (segment (start 93.6752 63.8556) (end 93.6752 56.2864) (width 0.75) (layer "B.Cu") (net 6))
 (segment (start 96.774 64.6176) (end 94.4372 64.6176) (width 0.75) (layer "B.Cu") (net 6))
 (segment (start 150.0124 62.8904) (end 151.3232 61.5796) (width 0.75) (layer "B.Cu") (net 6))
 (segment (start 145.6436 62.8904) (end 150.0124 62.8904) (width 0.75) (layer "B.Cu") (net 6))
 (segment (start 144.272 61.5188) (end 145.6436 62.8904) (width 0.75) (layer "B.Cu") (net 6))
 (segment (start 95.9104 54.0512) (end 142.24 54.0512) (width 0.75) (layer "B.Cu") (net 6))
 (segment (start 93.6244 73.4568) (end 97.6884 77.5208) (width 0.75) (layer "B.Cu") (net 4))
 (segment (start 160.274 77.5208) (end 163.068 74.7268) (width 0.75) (layer "B.Cu") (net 4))
 (segment (start 160.6196 61.5796) (end 160.6196 63.51) (width 0.75) (layer "B.Cu") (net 4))
 (segment (start 94.8436 67.1576) (end 93.6244 68.3768) (width 0.75) (layer "B.Cu") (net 4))
 (segment (start 93.6244 68.3768) (end 93.6244 73.4568) (width 0.75) (layer "B.Cu") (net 4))
 (segment (start 163.068 74.7268) (end 163.068 62.2808) (width 0.75) (layer "B.Cu") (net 4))
 (segment (start 96.774 67.1576) (end 94.8436 67.1576) (width 0.75) (layer "B.Cu") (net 4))
 (segment (start 141.3764 64.2112) (end 137.4648 60.2996) (width 0.75) (layer "B.Cu") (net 4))
 (segment (start 97.6884 77.5208) (end 160.274 77.5208) (width 0.75) (layer "B.Cu") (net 4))
 (segment (start 163.068 62.2808) (end 162.3668 61.5796) (width 0.75) (layer "B.Cu") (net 4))
 (segment (start 160.6196 63.51) (end 159.9184 64.2112) (width 0.75) (layer "B.Cu") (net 4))
 (segment (start 159.9184 64.2112) (end 141.3764 64.2112) (width 0.75) (layer "B.Cu") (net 4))
 (segment (start 162.3668 61.5796) (end 160.6196 61.5796) (width 0.75) (layer "B.Cu") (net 4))
 (segment (start 160.6196 72.3492) (end 160.6196 69.1996) (width 0.75) (layer "B.Cu") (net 9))
 (segment (start 97.79 69.6976) (end 104.1908 76.0984) (width 0.75) (layer "B.Cu") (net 9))
 (segment (start 104.1908 76.0984) (end 156.8704 76.0984) (width 0.75) (layer "B.Cu") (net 9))
 (segment (start 96.774 69.6976) (end 97.79 69.6976) (width 0.75) (layer "B.Cu") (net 9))
 (segment (start 156.8704 76.0984) (end 160.6196 72.3492) (width 0.75) (layer "B.Cu") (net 9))
 (segment (start 155.0924 56.642) (end 158.0796 59.6292) (width 0.75) (layer "B.Cu") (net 3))
 (segment (start 158.0796 59.6292) (end 158.0796 61.5796) (width 0.75) (layer "B.Cu") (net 3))
 (segment (start 147.6248 56.642) (end 155.0924 56.642) (width 0.75) (layer "B.Cu") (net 3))
 (segment (start 147.6248 56.642) (end 147.6248 60.2996) (width 0.75) (layer "B.Cu") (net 3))
 (segment (start 154.4828 72.7456) (end 146.6596 72.7456) (width 0.75) (layer "B.Cu") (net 7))
 (segment (start 146.6596 72.7456) (end 146.6596 69.088) (width 0.75) (layer "B.Cu") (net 7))
 (segment (start 146.6596 69.088) (end 146.7612 68.9864) (width 0.75) (layer "B.Cu") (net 7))
 (segment (start 146.7612 72.9996) (end 146.6596 73.1012) (width 0.75) (layer "B.Cu") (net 7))
 (segment (start 155.5396 71.6888) (end 155.5396 69.1996) (width 0.75) (layer "B.Cu") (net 7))
 (segment (start 155.5396 71.6888) (end 154.4828 72.7456) (width 0.75) (layer "B.Cu") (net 7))
 (segment (start 146.7612 72.136) (end 146.6596 72.2376) (width 0.75) (layer "B.Cu") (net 7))
 (segment (start 117.8306 64.008) (end 113.9444 64.008) (width 0.75) (layer "B.Cu") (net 1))
 (segment (start 122.6566 61.468) (end 122.6566 58.674) (width 0.75) (layer "B.Cu") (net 1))
 (segment (start 113.8936 64.0588) (end 111.2012 61.3664) (width 0.75) (layer "B.Cu") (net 1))
 (segment (start 117.8306 64.008) (end 120.1166 64.008) (width 0.75) (layer "B.Cu") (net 1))
 (segment (start 113.9444 64.008) (end 113.8936 64.0588) (width 0.75) (layer "B.Cu") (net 1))
 (segment (start 111.2012 61.3664) (end 111.2012 58.8264) (width 0.75) (layer "B.Cu") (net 1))
 (segment (start 120.1166 64.008) (end 122.6566 61.468) (width 0.75) (layer "B.Cu") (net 1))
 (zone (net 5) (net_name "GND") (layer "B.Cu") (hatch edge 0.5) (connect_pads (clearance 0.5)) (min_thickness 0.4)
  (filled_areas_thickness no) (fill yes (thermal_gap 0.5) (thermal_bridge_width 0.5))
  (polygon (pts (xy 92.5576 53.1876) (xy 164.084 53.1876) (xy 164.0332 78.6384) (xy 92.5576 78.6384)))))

